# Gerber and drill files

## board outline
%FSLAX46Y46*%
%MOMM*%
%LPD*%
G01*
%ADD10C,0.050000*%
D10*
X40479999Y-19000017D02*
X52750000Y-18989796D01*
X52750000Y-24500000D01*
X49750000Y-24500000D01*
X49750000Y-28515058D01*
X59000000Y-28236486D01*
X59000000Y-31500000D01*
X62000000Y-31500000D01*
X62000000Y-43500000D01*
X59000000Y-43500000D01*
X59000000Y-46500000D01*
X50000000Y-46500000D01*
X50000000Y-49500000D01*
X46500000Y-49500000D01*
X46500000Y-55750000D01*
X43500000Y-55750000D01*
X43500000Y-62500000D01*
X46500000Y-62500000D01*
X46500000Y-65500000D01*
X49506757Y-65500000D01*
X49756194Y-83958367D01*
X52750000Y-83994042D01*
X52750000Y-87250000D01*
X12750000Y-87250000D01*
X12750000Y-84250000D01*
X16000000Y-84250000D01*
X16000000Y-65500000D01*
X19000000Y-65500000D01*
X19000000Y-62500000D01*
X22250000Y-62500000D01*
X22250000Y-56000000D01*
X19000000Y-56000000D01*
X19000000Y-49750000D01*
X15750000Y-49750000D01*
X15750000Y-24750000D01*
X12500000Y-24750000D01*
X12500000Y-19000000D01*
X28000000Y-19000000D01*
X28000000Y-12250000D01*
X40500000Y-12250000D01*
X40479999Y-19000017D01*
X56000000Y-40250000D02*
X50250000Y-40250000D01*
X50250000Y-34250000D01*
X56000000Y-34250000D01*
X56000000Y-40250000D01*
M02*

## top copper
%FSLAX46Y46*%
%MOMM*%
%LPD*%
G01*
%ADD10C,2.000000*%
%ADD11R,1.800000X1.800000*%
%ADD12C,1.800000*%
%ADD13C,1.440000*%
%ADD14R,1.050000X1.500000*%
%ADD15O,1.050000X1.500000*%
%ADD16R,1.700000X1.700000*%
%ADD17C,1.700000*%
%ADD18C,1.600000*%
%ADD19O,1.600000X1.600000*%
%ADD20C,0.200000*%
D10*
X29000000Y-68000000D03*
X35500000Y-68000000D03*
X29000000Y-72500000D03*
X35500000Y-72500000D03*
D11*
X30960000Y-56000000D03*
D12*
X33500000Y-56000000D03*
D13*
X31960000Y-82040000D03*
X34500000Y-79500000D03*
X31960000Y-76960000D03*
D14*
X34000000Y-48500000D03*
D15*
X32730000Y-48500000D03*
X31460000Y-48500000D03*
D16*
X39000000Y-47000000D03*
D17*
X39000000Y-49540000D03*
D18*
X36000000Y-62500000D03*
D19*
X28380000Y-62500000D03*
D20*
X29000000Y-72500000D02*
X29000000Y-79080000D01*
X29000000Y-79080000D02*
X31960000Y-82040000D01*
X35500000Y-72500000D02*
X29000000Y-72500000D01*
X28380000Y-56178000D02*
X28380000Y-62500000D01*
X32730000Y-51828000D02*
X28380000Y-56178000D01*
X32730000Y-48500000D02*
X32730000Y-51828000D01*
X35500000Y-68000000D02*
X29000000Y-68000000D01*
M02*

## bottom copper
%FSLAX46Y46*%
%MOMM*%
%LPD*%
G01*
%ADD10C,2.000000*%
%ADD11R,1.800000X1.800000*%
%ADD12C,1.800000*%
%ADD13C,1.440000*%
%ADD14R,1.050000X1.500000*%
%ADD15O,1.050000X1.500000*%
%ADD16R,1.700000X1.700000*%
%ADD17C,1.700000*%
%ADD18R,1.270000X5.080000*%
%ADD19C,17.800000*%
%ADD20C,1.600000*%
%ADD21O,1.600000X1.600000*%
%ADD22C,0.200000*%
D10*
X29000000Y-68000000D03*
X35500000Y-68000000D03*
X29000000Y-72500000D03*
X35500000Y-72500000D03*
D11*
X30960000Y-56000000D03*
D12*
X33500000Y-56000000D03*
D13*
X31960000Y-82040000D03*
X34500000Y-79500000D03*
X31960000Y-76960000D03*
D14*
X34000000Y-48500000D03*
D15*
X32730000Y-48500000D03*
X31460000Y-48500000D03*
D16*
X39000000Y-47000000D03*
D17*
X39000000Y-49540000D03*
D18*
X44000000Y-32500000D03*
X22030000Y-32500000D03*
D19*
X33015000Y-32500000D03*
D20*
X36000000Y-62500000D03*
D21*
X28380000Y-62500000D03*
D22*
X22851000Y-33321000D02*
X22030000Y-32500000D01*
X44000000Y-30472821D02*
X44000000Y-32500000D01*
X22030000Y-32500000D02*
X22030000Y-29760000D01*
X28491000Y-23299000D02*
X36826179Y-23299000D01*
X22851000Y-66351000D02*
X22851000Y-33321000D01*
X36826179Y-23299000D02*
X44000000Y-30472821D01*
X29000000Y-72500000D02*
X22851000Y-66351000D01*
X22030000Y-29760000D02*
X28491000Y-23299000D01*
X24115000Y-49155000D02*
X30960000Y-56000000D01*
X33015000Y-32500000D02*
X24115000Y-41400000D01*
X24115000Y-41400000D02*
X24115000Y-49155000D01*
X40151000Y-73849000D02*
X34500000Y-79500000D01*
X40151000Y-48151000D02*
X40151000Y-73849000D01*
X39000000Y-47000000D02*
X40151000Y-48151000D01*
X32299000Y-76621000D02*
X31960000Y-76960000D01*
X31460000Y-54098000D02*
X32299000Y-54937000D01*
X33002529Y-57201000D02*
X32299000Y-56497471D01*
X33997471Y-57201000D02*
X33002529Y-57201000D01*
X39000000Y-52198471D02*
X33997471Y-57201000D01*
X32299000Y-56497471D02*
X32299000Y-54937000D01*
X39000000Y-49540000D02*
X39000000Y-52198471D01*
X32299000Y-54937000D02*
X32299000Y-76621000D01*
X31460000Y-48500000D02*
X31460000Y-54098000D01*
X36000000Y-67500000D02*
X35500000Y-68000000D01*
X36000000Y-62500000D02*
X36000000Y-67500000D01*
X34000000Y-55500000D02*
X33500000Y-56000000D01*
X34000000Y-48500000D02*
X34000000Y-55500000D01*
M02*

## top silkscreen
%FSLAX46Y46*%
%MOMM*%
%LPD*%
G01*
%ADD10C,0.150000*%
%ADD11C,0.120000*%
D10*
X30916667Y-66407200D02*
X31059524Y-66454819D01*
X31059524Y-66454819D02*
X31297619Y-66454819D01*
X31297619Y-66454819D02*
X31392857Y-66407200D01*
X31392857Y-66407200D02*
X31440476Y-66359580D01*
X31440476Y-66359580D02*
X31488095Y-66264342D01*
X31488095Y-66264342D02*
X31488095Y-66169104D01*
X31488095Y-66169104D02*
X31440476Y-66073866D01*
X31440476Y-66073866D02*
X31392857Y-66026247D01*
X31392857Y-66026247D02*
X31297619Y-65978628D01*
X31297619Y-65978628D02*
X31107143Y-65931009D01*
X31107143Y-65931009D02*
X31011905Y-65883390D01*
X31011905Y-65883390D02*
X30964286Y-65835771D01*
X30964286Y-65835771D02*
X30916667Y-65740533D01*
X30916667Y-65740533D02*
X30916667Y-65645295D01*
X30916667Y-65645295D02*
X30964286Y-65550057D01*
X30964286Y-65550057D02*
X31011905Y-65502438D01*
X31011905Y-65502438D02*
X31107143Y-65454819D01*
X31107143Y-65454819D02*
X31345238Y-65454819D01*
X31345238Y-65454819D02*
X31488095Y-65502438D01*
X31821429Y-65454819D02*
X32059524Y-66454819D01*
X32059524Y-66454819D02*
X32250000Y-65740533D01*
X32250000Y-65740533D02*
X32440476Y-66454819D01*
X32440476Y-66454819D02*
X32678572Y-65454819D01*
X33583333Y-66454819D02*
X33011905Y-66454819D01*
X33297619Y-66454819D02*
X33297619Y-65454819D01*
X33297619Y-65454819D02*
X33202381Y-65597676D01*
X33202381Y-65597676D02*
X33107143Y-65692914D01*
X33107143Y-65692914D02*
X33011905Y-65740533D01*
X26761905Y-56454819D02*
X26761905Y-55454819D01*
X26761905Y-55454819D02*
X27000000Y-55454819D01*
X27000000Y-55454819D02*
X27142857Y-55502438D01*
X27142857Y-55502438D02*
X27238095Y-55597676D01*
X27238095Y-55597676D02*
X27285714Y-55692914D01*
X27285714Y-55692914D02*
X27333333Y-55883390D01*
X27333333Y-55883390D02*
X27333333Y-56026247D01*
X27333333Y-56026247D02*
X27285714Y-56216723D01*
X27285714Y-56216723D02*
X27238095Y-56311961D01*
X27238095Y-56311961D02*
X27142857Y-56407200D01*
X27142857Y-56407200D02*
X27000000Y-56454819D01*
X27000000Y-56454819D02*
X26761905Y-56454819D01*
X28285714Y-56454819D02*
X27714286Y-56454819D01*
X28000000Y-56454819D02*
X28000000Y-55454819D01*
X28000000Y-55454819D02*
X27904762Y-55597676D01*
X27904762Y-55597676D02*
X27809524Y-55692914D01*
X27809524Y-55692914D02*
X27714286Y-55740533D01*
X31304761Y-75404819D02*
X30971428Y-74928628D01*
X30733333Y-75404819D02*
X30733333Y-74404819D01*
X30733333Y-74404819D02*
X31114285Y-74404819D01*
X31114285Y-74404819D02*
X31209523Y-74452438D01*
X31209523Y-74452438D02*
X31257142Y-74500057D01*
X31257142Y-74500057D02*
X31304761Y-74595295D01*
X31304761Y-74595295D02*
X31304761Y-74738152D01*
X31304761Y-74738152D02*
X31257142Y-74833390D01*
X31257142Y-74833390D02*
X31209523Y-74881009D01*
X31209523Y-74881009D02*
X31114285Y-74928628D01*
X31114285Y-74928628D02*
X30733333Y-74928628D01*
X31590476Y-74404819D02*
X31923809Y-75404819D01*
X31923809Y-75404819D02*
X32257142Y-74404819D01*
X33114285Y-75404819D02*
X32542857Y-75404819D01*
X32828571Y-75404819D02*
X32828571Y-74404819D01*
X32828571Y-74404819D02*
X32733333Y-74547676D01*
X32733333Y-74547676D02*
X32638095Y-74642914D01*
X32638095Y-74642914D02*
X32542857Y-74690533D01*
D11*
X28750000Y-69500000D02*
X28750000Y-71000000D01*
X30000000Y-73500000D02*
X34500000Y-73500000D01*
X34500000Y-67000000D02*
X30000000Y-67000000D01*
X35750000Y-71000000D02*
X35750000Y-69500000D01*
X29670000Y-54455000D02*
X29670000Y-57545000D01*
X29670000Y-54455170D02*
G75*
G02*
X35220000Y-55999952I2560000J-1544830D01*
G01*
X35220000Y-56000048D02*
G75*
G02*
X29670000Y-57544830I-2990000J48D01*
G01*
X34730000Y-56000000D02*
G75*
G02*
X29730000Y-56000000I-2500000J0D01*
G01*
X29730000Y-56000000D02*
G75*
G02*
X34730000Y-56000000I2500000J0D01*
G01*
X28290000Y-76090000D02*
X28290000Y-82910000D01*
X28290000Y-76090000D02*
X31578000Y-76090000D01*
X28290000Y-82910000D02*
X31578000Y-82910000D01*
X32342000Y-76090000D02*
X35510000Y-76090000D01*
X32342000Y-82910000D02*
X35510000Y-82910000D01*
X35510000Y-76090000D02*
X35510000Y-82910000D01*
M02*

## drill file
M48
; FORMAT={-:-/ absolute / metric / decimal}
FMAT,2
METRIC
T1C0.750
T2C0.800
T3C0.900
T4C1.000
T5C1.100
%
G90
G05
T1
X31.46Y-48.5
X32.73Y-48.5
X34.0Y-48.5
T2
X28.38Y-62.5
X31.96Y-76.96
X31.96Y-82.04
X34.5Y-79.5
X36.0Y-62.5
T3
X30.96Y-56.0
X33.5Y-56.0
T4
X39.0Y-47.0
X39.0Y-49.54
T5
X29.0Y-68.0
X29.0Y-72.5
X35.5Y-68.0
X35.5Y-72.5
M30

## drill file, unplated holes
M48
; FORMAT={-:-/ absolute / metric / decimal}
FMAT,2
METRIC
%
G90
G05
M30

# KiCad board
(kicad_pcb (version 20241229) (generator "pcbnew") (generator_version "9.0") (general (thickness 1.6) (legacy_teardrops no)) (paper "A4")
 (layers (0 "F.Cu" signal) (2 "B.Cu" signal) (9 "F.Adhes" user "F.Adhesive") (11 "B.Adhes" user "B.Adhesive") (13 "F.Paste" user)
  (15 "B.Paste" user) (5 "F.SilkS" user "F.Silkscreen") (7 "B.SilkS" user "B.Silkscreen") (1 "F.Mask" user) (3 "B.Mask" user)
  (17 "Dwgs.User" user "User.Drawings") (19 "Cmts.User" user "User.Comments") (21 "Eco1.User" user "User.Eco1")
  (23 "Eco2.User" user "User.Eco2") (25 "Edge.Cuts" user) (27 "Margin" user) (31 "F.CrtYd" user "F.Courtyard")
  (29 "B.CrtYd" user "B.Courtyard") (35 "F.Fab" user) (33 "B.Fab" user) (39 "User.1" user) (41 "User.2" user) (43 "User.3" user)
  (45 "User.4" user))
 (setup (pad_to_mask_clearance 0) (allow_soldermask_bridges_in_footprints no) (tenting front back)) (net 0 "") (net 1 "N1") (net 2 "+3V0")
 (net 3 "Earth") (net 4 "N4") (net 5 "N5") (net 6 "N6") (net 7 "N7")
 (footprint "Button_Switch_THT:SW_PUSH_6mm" (layer "F.Cu") (at 29 68)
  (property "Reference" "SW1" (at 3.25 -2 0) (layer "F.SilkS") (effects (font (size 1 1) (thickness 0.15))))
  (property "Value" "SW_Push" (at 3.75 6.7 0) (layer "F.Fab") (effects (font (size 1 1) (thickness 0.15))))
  (fp_line (start -0.25 1.5) (end -0.25 3) (stroke (width 0.12) (type solid)) (layer "F.SilkS"))
  (fp_line (start 1 5.5) (end 5.5 5.5) (stroke (width 0.12) (type solid)) (layer "F.SilkS"))
  (fp_line (start 5.5 -1) (end 1 -1) (stroke (width 0.12) (type solid)) (layer "F.SilkS"))
  (fp_line (start 6.75 3) (end 6.75 1.5) (stroke (width 0.12) (type solid)) (layer "F.SilkS"))
  (pad "1" thru_hole circle (at 0 0 90) (size 2 2) (drill 1.1) (layers "*.Cu" "*.Mask") (remove_unused_layers no) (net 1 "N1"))
  (pad "1" thru_hole circle (at 6.5 0 90) (size 2 2) (drill 1.1) (layers "*.Cu" "*.Mask") (remove_unused_layers no) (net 1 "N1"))
  (pad "2" thru_hole circle (at 0 4.5 90) (size 2 2) (drill 1.1) (layers "*.Cu" "*.Mask") (remove_unused_layers no) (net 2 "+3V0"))
  (pad "2" thru_hole circle (at 6.5 4.5 90) (size 2 2) (drill 1.1) (layers "*.Cu" "*.Mask") (remove_unused_layers no) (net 2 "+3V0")))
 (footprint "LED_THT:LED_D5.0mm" (layer "F.Cu") (at 30.96 56)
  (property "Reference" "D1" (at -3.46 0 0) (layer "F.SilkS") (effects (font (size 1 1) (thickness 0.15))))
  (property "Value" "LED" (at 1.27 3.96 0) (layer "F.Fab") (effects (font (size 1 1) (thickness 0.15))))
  (fp_line (start -1.29 -1.545) (end -1.29 1.545) (stroke (width 0.12) (type solid)) (layer "F.SilkS"))
  (fp_arc (start -1.29 -1.54483) (mid 2.071756 -2.880501) (end 4.26 -0.000048) (stroke (width 0.12) (type solid)) (layer "F.SilkS"))
  (fp_arc (start 4.26 0.000048) (mid 2.071756 2.880501) (end -1.29 1.54483) (stroke (width 0.12) (type solid)) (layer "F.SilkS"))
  (fp_circle (center 1.27 0) (end 3.77 0) (stroke (width 0.12) (type solid)) (fill no) (layer "F.SilkS"))
  (pad "1" thru_hole rect (at 0 0) (size 1.8 1.8) (drill 0.9) (layers "*.Cu" "*.Mask") (remove_unused_layers no) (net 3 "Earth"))
  (pad "2" thru_hole circle (at 2.54 0) (size 1.8 1.8) (drill 0.9) (layers "*.Cu" "*.Mask") (remove_unused_layers no) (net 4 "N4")))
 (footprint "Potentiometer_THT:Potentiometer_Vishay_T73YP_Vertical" (layer "F.Cu") (at 31.96 82.04)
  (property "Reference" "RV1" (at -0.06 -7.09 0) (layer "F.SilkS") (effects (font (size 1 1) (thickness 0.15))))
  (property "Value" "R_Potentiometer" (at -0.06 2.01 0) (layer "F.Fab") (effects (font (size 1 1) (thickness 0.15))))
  (fp_line (start -3.67 -5.95) (end -3.67 0.87) (stroke (width 0.12) (type solid)) (layer "F.SilkS"))
  (fp_line (start -3.67 -5.95) (end -0.382 -5.95) (stroke (width 0.12) (type solid)) (layer "F.SilkS"))
  (fp_line (start -3.67 0.87) (end -0.382 0.87) (stroke (width 0.12) (type solid)) (layer "F.SilkS"))
  (fp_line (start 0.382 -5.95) (end 3.55 -5.95) (stroke (width 0.12) (type solid)) (layer "F.SilkS"))
  (fp_line (start 0.382 0.87) (end 3.55 0.87) (stroke (width 0.12) (type solid)) (layer "F.SilkS"))
  (fp_line (start 3.55 -5.95) (end 3.55 0.87) (stroke (width 0.12) (type solid)) (layer "F.SilkS"))
  (pad "1" thru_hole circle (at 0 0) (size 1.44 1.44) (drill 0.8) (layers "*.Cu" "*.Mask") (remove_unused_layers no) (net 2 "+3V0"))
  (pad "2" thru_hole circle (at 2.54 -2.54) (size 1.44 1.44) (drill 0.8) (layers "*.Cu" "*.Mask") (remove_unused_layers no) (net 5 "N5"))
  (pad "3" thru_hole circle (at 0 -5.08) (size 1.44 1.44) (drill 0.8) (layers "*.Cu" "*.Mask") (remove_unused_layers no) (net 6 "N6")))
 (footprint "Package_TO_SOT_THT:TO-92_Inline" (layer "B.Cu") (at 34 48.5 180)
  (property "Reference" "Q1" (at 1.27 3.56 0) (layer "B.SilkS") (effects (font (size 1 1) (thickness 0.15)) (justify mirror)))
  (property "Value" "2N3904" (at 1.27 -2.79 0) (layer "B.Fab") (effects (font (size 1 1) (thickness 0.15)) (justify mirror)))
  (pad "1" thru_hole rect (at 0 0 180) (size 1.05 1.5) (drill 0.75) (layers "*.Cu" "*.Mask") (remove_unused_layers no) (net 4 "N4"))
  (pad "2" thru_hole oval (at 1.27 0 180) (size 1.05 1.5) (drill 0.75) (layers "*.Cu" "*.Mask") (remove_unused_layers no) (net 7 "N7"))
  (pad "3" thru_hole oval (at 2.54 0 180) (size 1.05 1.5) (drill 0.75) (layers "*.Cu" "*.Mask") (remove_unused_layers no) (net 6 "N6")))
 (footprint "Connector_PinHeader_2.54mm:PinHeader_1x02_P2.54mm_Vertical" (layer "B.Cu") (at 39 47 180)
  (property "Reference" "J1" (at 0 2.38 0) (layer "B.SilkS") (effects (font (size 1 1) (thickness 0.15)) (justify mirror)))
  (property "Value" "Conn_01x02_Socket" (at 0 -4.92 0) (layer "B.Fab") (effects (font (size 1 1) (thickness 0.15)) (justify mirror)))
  (pad "1" thru_hole rect (at 0 0 180) (size 1.7 1.7) (drill 1) (layers "*.Cu" "*.Mask") (remove_unused_layers no) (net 5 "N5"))
  (pad "2" thru_hole circle (at 0 -2.54 180) (size 1.7 1.7) (drill 1) (layers "*.Cu" "*.Mask") (remove_unused_layers no) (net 6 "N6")))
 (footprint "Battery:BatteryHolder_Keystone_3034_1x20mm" (layer "B.Cu") (at 33.015 32.5 180)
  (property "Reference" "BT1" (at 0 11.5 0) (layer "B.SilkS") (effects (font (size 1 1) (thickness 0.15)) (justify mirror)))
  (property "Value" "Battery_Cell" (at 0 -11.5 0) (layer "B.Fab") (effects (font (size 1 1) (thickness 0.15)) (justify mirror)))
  (pad "1" smd rect (at -10.985 0 180) (size 1.27 5.08) (layers "B.Cu" "B.Mask" "B.Paste") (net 2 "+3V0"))
  (pad "1" smd rect (at 10.985 0 180) (size 1.27 5.08) (layers "B.Cu" "B.Mask" "B.Paste") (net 2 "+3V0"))
  (pad "2" smd circle (at 0 0 180) (size 17.8 17.8) (layers "B.Cu" "B.Mask") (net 3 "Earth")))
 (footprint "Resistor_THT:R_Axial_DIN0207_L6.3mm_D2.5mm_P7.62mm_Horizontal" (layer "B.Cu") (at 36 62.5 180)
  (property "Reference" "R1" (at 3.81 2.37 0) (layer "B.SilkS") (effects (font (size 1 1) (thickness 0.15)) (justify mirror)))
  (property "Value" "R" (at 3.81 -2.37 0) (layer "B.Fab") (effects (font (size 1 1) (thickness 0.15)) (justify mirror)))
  (pad "1" thru_hole circle (at 0 0 180) (size 1.6 1.6) (drill 0.8) (layers "*.Cu" "*.Mask") (remove_unused_layers no) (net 1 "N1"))
  (pad "2" thru_hole oval (at 7.62 0 180) (size 1.6 1.6) (drill 0.8) (layers "*.Cu" "*.Mask") (remove_unused_layers no) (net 7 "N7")))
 (gr_poly
  (pts (xy 28 12.25) (xy 28 19) (xy 12.5 19) (xy 12.5 24.75) (xy 15.75 24.75) (xy 15.75 49.75) (xy 19 49.75) (xy 19 56) (xy 22.25 56)
   (xy 22.25 62.5) (xy 19 62.5) (xy 19 65.5) (xy 16 65.5) (xy 16 84.25) (xy 12.75 84.25) (xy 12.75 87.25) (xy 52.75 87.25)
   (xy 52.75 83.994042) (xy 49.756194 83.958367) (xy 49.506757 65.5) (xy 46.5 65.5) (xy 46.5 62.5) (xy 43.5 62.5) (xy 43.5 55.75)
   (xy 46.5 55.75) (xy 46.5 49.5) (xy 50 49.5) (xy 50 46.5) (xy 59 46.5) (xy 59 43.5) (xy 62 43.5) (xy 62 31.5) (xy 59 31.5)
   (xy 59 28.236486) (xy 49.75 28.515058) (xy 49.75 24.5) (xy 52.75 24.5) (xy 52.75 18.989796) (xy 40.479999 19.000017) (xy 40.5 12.25))
  (stroke (width 0.05) (type solid)) (fill no) (layer "Edge.Cuts"))
 (gr_poly
  (pts (xy 50.25 34.25) (xy 50.25 40.25) (xy 56 40.25) (xy 56 34.25)) (stroke (width 0.05) (type solid)) (fill no) (layer "Edge.Cuts"))
 (segment (start 29 72.5) (end 29 79.08) (width 0.2) (layer "F.Cu") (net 2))
 (segment (start 29 79.08) (end 31.96 82.04) (width 0.2) (layer "F.Cu") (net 2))
 (segment (start 35.5 72.5) (end 29 72.5) (width 0.2) (layer "F.Cu") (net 2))
 (segment (start 22.851 33.321) (end 22.03 32.5) (width 0.2) (layer "B.Cu") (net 2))
 (segment (start 44 30.472821) (end 44 32.5) (width 0.2) (layer "B.Cu") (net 2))
 (segment (start 22.03 32.5) (end 22.03 29.76) (width 0.2) (layer "B.Cu") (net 2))
 (segment (start 28.491 23.299) (end 36.826179 23.299) (width 0.2) (layer "B.Cu") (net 2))
 (segment (start 22.851 66.351) (end 22.851 33.321) (width 0.2) (layer "B.Cu") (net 2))
 (segment (start 36.826179 23.299) (end 44 30.472821) (width 0.2) (layer "B.Cu") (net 2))
 (segment (start 29 72.5) (end 22.851 66.351) (width 0.2) (layer "B.Cu") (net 2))
 (segment (start 22.03 29.76) (end 28.491 23.299) (width 0.2) (layer "B.Cu") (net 2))
 (segment (start 24.115 49.155) (end 30.96 56) (width 0.2) (layer "B.Cu") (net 3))
 (segment (start 33.015 32.5) (end 24.115 41.4) (width 0.2) (layer "B.Cu") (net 3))
 (segment (start 24.115 41.4) (end 24.115 49.155) (width 0.2) (layer "B.Cu") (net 3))
 (segment (start 40.151 73.849) (end 34.5 79.5) (width 0.2) (layer "B.Cu") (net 5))
 (segment (start 40.151 48.151) (end 40.151 73.849) (width 0.2) (layer "B.Cu") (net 5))
 (segment (start 39 47) (end 40.151 48.151) (width 0.2) (layer "B.Cu") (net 5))
 (segment (start 32.299 76.621) (end 31.96 76.96) (width 0.2) (layer "B.Cu") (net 6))
 (segment (start 31.46 54.098) (end 32.299 54.937) (width 0.2) (layer "B.Cu") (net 6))
 (segment (start 33.002529 57.201) (end 32.299 56.497471) (width 0.2) (layer "B.Cu") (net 6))
 (segment (start 33.997471 57.201) (end 33.002529 57.201) (width 0.2) (layer "B.Cu") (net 6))
 (segment (start 39 52.198471) (end 33.997471 57.201) (width 0.2) (layer "B.Cu") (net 6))
 (segment (start 32.299 56.497471) (end 32.299 54.937) (width 0.2) (layer "B.Cu") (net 6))
 (segment (start 39 49.54) (end 39 52.198471) (width 0.2) (layer "B.Cu") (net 6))
 (segment (start 32.299 54.937) (end 32.299 76.621) (width 0.2) (layer "B.Cu") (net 6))
 (segment (start 31.46 48.5) (end 31.46 54.098) (width 0.2) (layer "B.Cu") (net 6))
 (segment (start 28.38 56.178) (end 28.38 62.5) (width 0.2) (layer "F.Cu") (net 7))
 (segment (start 32.73 51.828) (end 28.38 56.178) (width 0.2) (layer "F.Cu") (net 7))
 (segment (start 32.73 48.5) (end 32.73 51.828) (width 0.2) (layer "F.Cu") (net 7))
 (segment (start 35.5 68) (end 29 68) (width 0.2) (layer "F.Cu") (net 1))
 (segment (start 36 67.5) (end 35.5 68) (width 0.2) (layer "B.Cu") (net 1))
 (segment (start 36 62.5) (end 36 67.5) (width 0.2) (layer "B.Cu") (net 1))
 (segment (start 34 55.5) (end 33.5 56) (width 0.2) (layer "B.Cu") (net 4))
 (segment (start 34 48.5) (end 34 55.5) (width 0.2) (layer "B.Cu") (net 4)))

